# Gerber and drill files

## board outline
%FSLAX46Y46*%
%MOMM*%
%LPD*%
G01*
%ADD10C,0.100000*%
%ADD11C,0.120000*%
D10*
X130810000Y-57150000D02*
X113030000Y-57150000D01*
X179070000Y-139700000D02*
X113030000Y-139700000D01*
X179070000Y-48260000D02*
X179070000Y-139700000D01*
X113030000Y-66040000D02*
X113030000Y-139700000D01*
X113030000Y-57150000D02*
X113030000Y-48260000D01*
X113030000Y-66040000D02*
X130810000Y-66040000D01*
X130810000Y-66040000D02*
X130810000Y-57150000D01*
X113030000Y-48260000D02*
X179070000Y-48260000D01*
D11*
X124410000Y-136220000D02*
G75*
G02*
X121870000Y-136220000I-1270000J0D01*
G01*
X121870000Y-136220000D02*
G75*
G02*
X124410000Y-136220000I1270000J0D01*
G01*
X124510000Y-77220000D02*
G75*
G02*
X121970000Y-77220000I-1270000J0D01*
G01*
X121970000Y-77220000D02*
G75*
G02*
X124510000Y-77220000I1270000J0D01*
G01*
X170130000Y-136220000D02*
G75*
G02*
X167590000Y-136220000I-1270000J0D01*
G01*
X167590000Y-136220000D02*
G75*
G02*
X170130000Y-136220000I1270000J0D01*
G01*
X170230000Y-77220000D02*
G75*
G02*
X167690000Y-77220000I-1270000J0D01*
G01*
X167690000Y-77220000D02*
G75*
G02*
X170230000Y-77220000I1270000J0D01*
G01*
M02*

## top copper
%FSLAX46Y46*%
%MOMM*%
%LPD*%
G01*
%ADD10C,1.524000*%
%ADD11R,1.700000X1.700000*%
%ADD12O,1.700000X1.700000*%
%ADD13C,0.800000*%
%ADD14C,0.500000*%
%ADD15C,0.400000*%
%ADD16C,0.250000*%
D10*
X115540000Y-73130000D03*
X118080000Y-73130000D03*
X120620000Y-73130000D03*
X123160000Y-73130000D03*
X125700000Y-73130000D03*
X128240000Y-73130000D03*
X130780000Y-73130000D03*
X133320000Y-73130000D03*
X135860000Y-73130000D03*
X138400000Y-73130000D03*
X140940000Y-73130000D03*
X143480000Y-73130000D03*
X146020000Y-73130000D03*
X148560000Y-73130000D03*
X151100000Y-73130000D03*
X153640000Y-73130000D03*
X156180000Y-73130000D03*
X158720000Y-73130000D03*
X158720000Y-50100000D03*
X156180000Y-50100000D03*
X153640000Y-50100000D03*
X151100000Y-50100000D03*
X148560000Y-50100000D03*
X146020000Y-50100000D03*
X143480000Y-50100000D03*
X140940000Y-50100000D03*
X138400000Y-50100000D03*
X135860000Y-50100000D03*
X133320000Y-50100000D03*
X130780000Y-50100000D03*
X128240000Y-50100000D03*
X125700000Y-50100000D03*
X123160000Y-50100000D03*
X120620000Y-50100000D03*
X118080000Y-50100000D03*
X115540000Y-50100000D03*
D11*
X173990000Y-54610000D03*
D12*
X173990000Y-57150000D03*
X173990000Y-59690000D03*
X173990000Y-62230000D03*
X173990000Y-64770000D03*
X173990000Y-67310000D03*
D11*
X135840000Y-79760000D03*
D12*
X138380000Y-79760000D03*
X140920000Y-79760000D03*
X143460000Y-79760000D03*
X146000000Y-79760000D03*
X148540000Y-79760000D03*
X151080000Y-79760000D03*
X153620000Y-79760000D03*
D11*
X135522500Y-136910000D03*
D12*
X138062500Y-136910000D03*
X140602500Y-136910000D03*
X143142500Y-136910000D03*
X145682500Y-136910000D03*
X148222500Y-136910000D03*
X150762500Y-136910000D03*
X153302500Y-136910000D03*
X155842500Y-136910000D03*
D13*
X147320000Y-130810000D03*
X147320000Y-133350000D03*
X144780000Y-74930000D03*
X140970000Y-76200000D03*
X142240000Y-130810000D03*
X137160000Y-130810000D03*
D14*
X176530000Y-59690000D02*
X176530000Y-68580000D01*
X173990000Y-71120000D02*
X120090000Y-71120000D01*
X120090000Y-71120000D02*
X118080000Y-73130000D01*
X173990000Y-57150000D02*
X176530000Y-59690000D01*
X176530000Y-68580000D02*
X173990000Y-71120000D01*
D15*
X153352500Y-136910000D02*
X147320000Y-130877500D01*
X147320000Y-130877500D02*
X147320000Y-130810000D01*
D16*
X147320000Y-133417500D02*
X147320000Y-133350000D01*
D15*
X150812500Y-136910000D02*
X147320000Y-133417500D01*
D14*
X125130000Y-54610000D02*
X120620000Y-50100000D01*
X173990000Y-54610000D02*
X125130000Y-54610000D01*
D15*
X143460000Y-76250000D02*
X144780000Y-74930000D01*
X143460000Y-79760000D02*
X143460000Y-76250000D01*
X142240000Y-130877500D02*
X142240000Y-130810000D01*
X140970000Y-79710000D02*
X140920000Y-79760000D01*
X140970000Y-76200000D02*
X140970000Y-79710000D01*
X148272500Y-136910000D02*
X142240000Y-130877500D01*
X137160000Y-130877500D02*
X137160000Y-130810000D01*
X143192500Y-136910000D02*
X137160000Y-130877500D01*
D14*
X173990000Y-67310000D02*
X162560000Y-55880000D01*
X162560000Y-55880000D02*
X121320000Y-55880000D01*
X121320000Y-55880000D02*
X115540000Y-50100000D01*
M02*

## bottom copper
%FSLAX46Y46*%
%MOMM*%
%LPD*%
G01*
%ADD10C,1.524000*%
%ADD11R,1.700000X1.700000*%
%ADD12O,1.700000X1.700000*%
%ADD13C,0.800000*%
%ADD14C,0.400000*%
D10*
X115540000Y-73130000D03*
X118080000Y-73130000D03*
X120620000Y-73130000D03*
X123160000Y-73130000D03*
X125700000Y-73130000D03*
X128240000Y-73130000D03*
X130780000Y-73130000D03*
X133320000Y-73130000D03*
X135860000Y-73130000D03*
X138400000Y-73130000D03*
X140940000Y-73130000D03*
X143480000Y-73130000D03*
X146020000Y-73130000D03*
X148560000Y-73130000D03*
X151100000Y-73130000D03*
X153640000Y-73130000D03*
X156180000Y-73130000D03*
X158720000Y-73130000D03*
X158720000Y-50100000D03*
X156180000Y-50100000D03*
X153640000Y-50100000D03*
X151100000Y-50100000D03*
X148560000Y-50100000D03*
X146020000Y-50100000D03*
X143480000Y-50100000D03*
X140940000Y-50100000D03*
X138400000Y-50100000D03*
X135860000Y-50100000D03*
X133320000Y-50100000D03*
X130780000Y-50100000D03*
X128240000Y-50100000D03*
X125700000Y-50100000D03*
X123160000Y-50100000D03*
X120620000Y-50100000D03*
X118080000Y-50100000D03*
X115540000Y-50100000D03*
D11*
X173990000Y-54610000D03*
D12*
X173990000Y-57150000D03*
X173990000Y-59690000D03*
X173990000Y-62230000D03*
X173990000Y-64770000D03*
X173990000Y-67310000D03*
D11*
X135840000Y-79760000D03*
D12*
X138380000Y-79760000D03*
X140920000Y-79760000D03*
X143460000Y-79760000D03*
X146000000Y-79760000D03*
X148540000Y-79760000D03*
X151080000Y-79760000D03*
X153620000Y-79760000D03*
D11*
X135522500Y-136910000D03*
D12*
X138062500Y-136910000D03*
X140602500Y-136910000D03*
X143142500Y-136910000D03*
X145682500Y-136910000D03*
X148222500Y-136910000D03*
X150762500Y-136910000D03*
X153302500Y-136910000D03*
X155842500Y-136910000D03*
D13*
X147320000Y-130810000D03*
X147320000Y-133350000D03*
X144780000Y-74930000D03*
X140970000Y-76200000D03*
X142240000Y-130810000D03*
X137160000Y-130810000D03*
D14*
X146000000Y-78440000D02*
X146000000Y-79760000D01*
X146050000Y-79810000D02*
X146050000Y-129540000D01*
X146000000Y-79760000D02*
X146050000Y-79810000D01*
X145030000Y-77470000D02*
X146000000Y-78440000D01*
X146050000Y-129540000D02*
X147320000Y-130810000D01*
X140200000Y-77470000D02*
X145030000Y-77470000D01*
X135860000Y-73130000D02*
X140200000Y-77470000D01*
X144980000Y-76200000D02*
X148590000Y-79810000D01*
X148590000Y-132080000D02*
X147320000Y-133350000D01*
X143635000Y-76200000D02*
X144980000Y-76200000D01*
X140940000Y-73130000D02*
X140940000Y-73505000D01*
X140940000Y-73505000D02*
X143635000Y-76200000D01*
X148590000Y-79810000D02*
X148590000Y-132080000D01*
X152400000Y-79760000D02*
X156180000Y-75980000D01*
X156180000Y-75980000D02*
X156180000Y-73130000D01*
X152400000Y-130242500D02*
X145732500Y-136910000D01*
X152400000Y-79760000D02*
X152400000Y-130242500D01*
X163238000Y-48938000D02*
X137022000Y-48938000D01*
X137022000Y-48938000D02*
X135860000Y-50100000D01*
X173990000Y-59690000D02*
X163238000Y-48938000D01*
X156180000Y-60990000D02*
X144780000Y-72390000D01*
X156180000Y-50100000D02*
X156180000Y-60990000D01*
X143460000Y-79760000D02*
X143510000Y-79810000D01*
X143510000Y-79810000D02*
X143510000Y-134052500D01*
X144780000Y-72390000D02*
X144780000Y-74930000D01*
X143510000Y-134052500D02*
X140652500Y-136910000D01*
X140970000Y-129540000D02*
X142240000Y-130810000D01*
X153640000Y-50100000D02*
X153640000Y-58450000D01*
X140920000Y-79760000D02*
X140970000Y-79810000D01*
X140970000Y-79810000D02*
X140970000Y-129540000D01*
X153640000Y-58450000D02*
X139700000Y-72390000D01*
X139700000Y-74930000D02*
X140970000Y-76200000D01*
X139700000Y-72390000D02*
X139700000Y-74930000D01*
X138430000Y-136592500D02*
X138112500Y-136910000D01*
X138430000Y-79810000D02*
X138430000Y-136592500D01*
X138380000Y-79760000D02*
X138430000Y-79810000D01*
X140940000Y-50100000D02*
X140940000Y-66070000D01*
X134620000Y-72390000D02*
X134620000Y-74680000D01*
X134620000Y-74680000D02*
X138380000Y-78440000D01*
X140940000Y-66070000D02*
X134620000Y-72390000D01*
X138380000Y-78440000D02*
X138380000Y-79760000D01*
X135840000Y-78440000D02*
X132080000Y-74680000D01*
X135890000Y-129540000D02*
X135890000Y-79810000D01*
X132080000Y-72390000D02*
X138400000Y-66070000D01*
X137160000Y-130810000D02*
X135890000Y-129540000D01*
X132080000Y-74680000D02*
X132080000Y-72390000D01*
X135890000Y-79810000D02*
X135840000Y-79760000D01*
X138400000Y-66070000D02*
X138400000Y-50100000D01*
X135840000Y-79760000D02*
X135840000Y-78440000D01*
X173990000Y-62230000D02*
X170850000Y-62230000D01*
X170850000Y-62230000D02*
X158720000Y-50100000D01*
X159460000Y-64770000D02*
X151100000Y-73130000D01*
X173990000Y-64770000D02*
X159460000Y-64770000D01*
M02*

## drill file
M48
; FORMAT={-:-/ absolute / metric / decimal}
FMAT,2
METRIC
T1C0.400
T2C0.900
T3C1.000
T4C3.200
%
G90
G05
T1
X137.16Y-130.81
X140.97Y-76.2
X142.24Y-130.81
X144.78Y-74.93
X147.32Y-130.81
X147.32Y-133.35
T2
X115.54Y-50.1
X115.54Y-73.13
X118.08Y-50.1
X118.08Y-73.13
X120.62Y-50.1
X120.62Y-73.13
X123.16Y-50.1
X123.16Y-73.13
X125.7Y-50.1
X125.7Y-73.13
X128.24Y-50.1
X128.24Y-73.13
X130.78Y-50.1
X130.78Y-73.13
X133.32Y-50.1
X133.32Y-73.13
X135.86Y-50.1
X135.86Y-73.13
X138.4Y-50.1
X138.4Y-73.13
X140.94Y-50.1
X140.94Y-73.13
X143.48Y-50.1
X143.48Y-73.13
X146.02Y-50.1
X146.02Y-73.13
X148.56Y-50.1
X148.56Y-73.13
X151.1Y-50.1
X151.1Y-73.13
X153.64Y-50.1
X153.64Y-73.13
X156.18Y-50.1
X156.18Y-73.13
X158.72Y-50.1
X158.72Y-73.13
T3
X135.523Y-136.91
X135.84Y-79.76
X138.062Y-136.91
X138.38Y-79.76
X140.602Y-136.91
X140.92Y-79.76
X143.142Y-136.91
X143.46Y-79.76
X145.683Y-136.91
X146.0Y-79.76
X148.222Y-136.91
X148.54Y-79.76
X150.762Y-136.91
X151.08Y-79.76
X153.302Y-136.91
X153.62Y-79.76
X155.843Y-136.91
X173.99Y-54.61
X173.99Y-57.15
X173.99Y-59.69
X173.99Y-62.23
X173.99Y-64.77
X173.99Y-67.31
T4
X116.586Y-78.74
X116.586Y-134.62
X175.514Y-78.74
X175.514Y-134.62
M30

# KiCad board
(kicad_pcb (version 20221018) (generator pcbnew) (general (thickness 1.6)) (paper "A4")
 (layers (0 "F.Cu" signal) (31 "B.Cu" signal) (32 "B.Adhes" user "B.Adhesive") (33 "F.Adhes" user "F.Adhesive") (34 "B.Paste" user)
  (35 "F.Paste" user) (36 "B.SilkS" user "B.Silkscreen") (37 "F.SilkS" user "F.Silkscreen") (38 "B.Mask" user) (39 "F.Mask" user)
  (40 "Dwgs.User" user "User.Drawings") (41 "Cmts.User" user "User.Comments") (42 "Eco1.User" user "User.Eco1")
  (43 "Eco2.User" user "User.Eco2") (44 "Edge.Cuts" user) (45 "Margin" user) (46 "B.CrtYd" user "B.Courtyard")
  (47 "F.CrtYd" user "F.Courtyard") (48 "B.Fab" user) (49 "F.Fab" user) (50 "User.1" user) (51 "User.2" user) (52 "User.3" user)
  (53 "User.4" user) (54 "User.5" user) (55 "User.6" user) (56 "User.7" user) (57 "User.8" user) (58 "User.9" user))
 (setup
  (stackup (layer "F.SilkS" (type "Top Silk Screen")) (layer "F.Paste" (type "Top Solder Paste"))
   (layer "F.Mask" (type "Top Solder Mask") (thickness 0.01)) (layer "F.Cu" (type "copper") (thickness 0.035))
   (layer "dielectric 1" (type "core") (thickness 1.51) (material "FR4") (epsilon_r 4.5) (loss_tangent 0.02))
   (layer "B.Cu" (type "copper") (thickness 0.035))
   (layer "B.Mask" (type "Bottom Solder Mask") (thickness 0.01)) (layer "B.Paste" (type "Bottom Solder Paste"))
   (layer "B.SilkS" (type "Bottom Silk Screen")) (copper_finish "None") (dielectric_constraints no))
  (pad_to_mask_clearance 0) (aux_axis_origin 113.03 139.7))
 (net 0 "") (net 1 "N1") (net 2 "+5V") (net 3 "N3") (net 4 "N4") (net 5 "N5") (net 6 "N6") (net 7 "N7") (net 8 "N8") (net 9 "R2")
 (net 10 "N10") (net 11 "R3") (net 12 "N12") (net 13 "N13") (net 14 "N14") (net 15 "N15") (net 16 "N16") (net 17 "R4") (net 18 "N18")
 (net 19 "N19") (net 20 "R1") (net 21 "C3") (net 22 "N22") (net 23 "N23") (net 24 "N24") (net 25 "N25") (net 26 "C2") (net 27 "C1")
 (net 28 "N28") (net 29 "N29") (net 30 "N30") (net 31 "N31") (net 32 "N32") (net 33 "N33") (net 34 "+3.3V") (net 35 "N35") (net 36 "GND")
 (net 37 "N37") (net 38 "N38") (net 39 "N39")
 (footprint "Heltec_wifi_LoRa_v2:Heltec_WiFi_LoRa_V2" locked (layer "F.Cu") (at 140.94 61.615 90)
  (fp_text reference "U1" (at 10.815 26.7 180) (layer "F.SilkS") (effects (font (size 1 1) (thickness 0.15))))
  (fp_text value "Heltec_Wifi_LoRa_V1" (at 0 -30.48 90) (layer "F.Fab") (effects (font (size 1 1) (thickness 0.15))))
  (pad "1" thru_hole circle locked (at -11.515 -25.4 90) (size 1.524 1.524) (drill 0.9) (layers "*.Cu" "*.Mask") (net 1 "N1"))
  (pad "2" thru_hole circle locked (at -11.515 -22.86 90) (size 1.524 1.524) (drill 0.9) (layers "*.Cu" "*.Mask") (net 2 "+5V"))
  (pad "3" thru_hole circle locked (at -11.515 -20.32 90) (size 1.524 1.524) (drill 0.9) (layers "*.Cu" "*.Mask") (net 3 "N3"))
  (pad "4" thru_hole circle locked (at -11.515 -17.78 90) (size 1.524 1.524) (drill 0.9) (layers "*.Cu" "*.Mask") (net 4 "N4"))
  (pad "5" thru_hole circle locked (at -11.515 -15.24 90) (size 1.524 1.524) (drill 0.9) (layers "*.Cu" "*.Mask") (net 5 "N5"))
  (pad "6" thru_hole circle locked (at -11.515 -12.7 90) (size 1.524 1.524) (drill 0.9) (layers "*.Cu" "*.Mask") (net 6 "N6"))
  (pad "7" thru_hole circle locked (at -11.515 -10.16 90) (size 1.524 1.524) (drill 0.9) (layers "*.Cu" "*.Mask") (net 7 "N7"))
  (pad "8" thru_hole circle locked (at -11.515 -7.62 90) (size 1.524 1.524) (drill 0.9) (layers "*.Cu" "*.Mask") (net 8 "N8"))
  (pad "9" thru_hole circle locked (at -11.515 -5.08 90) (size 1.524 1.524) (drill 0.9) (layers "*.Cu" "*.Mask") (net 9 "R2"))
  (pad "10" thru_hole circle locked (at -11.515 -2.54 90) (size 1.524 1.524) (drill 0.9) (layers "*.Cu" "*.Mask") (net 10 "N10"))
  (pad "11" thru_hole circle locked (at -11.515 0 90) (size 1.524 1.524) (drill 0.9) (layers "*.Cu" "*.Mask") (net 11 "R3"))
  (pad "12" thru_hole circle locked (at -11.515 2.54 90) (size 1.524 1.524) (drill 0.9) (layers "*.Cu" "*.Mask") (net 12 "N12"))
  (pad "13" thru_hole circle locked (at -11.515 5.08 90) (size 1.524 1.524) (drill 0.9) (layers "*.Cu" "*.Mask") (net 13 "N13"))
  (pad "14" thru_hole circle locked (at -11.515 7.62 90) (size 1.524 1.524) (drill 0.9) (layers "*.Cu" "*.Mask") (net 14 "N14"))
  (pad "15" thru_hole circle locked (at -11.515 10.16 90) (size 1.524 1.524) (drill 0.9) (layers "*.Cu" "*.Mask") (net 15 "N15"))
  (pad "16" thru_hole circle locked (at -11.515 12.7 90) (size 1.524 1.524) (drill 0.9) (layers "*.Cu" "*.Mask") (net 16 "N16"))
  (pad "17" thru_hole circle locked (at -11.515 15.24 90) (size 1.524 1.524) (drill 0.9) (layers "*.Cu" "*.Mask") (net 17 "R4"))
  (pad "18" thru_hole circle locked (at -11.515 17.78 90) (size 1.524 1.524) (drill 0.9) (layers "*.Cu" "*.Mask") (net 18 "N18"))
  (pad "19" thru_hole circle locked (at 11.515 17.78 90) (size 1.524 1.524) (drill 0.9) (layers "*.Cu" "*.Mask") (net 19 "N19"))
  (pad "20" thru_hole circle locked (at 11.515 15.24 90) (size 1.524 1.524) (drill 0.9) (layers "*.Cu" "*.Mask") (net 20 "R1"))
  (pad "21" thru_hole circle locked (at 11.515 12.7 90) (size 1.524 1.524) (drill 0.9) (layers "*.Cu" "*.Mask") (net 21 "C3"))
  (pad "22" thru_hole circle locked (at 11.515 10.16 90) (size 1.524 1.524) (drill 0.9) (layers "*.Cu" "*.Mask") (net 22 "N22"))
  (pad "23" thru_hole circle locked (at 11.515 7.62 90) (size 1.524 1.524) (drill 0.9) (layers "*.Cu" "*.Mask") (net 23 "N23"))
  (pad "24" thru_hole circle locked (at 11.515 5.08 90) (size 1.524 1.524) (drill 0.9) (layers "*.Cu" "*.Mask") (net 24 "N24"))
  (pad "25" thru_hole circle locked (at 11.515 2.54 90) (size 1.524 1.524) (drill 0.9) (layers "*.Cu" "*.Mask") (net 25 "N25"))
  (pad "26" thru_hole circle locked (at 11.515 0 90) (size 1.524 1.524) (drill 0.9) (layers "*.Cu" "*.Mask") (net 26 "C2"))
  (pad "27" thru_hole circle locked (at 11.515 -2.54 90) (size 1.524 1.524) (drill 0.9) (layers "*.Cu" "*.Mask") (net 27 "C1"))
  (pad "28" thru_hole circle locked (at 11.515 -5.08 90) (size 1.524 1.524) (drill 0.9) (layers "*.Cu" "*.Mask") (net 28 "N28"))
  (pad "29" thru_hole circle locked (at 11.515 -7.62 90) (size 1.524 1.524) (drill 0.9) (layers "*.Cu" "*.Mask") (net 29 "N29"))
  (pad "30" thru_hole circle locked (at 11.515 -10.16 90) (size 1.524 1.524) (drill 0.9) (layers "*.Cu" "*.Mask") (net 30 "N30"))
  (pad "31" thru_hole circle locked (at 11.515 -12.7 90) (size 1.524 1.524) (drill 0.9) (layers "*.Cu" "*.Mask") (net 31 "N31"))
  (pad "32" thru_hole circle locked (at 11.515 -15.24 90) (size 1.524 1.524) (drill 0.9) (layers "*.Cu" "*.Mask") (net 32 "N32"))
  (pad "33" thru_hole circle locked (at 11.515 -17.78 90) (size 1.524 1.524) (drill 0.9) (layers "*.Cu" "*.Mask") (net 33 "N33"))
  (pad "34" thru_hole circle locked (at 11.515 -20.32 90) (size 1.524 1.524) (drill 0.9) (layers "*.Cu" "*.Mask") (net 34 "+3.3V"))
  (pad "35" thru_hole circle locked (at 11.515 -22.86 90) (size 1.524 1.524) (drill 0.9) (layers "*.Cu" "*.Mask") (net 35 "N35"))
  (pad "36" thru_hole circle locked (at 11.515 -25.4 90) (size 1.524 1.524) (drill 0.9) (layers "*.Cu" "*.Mask") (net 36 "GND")))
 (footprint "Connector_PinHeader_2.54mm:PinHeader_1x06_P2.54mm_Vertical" (layer "F.Cu") (at 173.99 54.61)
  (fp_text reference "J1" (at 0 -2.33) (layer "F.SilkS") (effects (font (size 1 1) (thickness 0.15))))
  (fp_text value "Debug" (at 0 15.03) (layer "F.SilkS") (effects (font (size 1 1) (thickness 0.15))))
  (pad "1" thru_hole rect (at 0 0) (size 1.7 1.7) (drill 1) (layers "*.Cu" "*.Mask") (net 34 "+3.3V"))
  (pad "2" thru_hole oval (at 0 2.54) (size 1.7 1.7) (drill 1) (layers "*.Cu" "*.Mask") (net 2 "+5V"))
  (pad "3" thru_hole oval (at 0 5.08) (size 1.7 1.7) (drill 1) (layers "*.Cu" "*.Mask") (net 28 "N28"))
  (pad "4" thru_hole oval (at 0 7.62) (size 1.7 1.7) (drill 1) (layers "*.Cu" "*.Mask") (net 19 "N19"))
  (pad "5" thru_hole oval (at 0 10.16) (size 1.7 1.7) (drill 1) (layers "*.Cu" "*.Mask") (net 15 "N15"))
  (pad "6" thru_hole oval (at 0 12.7) (size 1.7 1.7) (drill 1) (layers "*.Cu" "*.Mask") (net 36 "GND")))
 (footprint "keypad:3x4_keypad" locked (layer "F.Cu") (at 135.84 79.76)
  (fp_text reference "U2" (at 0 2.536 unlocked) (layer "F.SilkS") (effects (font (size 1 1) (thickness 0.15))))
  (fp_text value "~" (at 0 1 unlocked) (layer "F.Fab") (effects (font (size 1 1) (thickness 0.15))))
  (fp_circle (center -12.7 56.46) (end -11.43 56.46) (stroke (width 0.12) (type default)) (fill none) (layer "Edge.Cuts"))
  (fp_circle (center -12.6 -2.54) (end -12.6 -3.81) (stroke (width 0.12) (type default)) (fill none) (layer "Edge.Cuts"))
  (fp_circle (center 33.02 56.46) (end 34.29 56.46) (stroke (width 0.12) (type default)) (fill none) (layer "Edge.Cuts"))
  (fp_circle (center 33.12 -2.54) (end 31.85 -2.54) (stroke (width 0.12) (type default)) (fill none) (layer "Edge.Cuts"))
  (pad "A1" thru_hole rect locked (at 0 0 90) (size 1.7 1.7) (drill 1) (layers "*.Cu" "*.Mask") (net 27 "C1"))
  (pad "A2" thru_hole oval locked (at 2.54 0 90) (size 1.7 1.7) (drill 1) (layers "*.Cu" "*.Mask") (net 26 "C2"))
  (pad "A3" thru_hole oval locked (at 5.08 0 90) (size 1.7 1.7) (drill 1) (layers "*.Cu" "*.Mask") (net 21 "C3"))
  (pad "A4" thru_hole oval locked (at 7.62 0 90) (size 1.7 1.7) (drill 1) (layers "*.Cu" "*.Mask") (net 20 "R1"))
  (pad "A5" thru_hole oval locked (at 10.16 0 90) (size 1.7 1.7) (drill 1) (layers "*.Cu" "*.Mask") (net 9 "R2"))
  (pad "A6" thru_hole oval locked (at 12.7 0 90) (size 1.7 1.7) (drill 1) (layers "*.Cu" "*.Mask") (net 11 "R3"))
  (pad "A7" thru_hole oval locked (at 15.24 0 90) (size 1.7 1.7) (drill 1) (layers "*.Cu" "*.Mask") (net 17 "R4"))
  (pad "A8" thru_hole oval locked (at 17.78 0 90) (size 1.7 1.7) (drill 1) (layers "*.Cu" "*.Mask") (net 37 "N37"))
  (pad "B1" thru_hole rect locked (at -0.3175 57.15 90) (size 1.7 1.7) (drill 1) (layers "*.Cu" "*.Mask") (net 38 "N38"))
  (pad "B2" thru_hole oval locked (at 2.2225 57.15 90) (size 1.7 1.7) (drill 1) (layers "*.Cu" "*.Mask") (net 26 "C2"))
  (pad "B3" thru_hole oval locked (at 4.7625 57.15 90) (size 1.7 1.7) (drill 1) (layers "*.Cu" "*.Mask") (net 20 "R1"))
  (pad "B4" thru_hole oval locked (at 7.3025 57.15 90) (size 1.7 1.7) (drill 1) (layers "*.Cu" "*.Mask") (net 27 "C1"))
  (pad "B5" thru_hole oval locked (at 9.8425 57.15 90) (size 1.7 1.7) (drill 1) (layers "*.Cu" "*.Mask") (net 17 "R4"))
  (pad "B6" thru_hole oval locked (at 12.3825 57.15 90) (size 1.7 1.7) (drill 1) (layers "*.Cu" "*.Mask") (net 21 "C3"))
  (pad "B7" thru_hole oval locked (at 14.9225 57.15 90) (size 1.7 1.7) (drill 1) (layers "*.Cu" "*.Mask") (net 11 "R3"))
  (pad "B8" thru_hole oval locked (at 17.4625 57.15 90) (size 1.7 1.7) (drill 1) (layers "*.Cu" "*.Mask") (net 9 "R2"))
  (pad "B9" thru_hole oval locked (at 20.0025 57.15 90) (size 1.7 1.7) (drill 1) (layers "*.Cu" "*.Mask") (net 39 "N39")))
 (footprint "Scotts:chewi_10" (layer "F.Cu") (at 116.586 102.362 90)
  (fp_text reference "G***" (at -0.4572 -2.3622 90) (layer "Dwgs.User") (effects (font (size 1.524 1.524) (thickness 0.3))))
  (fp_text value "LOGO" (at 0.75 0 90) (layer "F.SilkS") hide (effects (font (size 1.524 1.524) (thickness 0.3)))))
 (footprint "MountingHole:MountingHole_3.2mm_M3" (layer "F.Cu") (at 116.586 134.62)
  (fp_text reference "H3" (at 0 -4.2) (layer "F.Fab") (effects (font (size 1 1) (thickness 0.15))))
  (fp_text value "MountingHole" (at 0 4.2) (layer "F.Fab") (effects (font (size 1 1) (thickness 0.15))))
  (pad "" np_thru_hole circle (at 0 0) (size 3.2 3.2) (drill 3.2) (layers "*.Cu" "*.Mask")))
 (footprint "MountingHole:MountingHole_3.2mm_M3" (layer "F.Cu") (at 116.586 78.74)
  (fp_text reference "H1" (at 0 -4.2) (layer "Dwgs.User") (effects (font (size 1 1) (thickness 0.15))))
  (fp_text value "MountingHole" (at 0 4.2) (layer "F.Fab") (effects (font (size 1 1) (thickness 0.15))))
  (pad "" np_thru_hole circle (at 0 0) (size 3.2 3.2) (drill 3.2) (layers "*.Cu" "*.Mask")))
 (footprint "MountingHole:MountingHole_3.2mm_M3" (layer "F.Cu") (at 175.514 78.74)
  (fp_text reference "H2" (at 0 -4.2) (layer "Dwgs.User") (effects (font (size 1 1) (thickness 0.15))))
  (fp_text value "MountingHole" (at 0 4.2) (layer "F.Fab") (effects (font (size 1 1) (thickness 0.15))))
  (pad "" np_thru_hole circle (at 0 0) (size 3.2 3.2) (drill 3.2) (layers "*.Cu" "*.Mask")))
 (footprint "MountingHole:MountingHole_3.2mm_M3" (layer "F.Cu") (at 175.514 134.62)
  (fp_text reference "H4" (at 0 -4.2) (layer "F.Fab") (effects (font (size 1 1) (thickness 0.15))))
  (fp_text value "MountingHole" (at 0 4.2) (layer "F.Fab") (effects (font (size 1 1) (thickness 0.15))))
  (pad "" np_thru_hole circle (at 0 0) (size 3.2 3.2) (drill 3.2) (layers "*.Cu" "*.Mask")))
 (gr_line (start 130.81 57.15) (end 113.03 57.15) (stroke (width 0.1) (type default)) (layer "Edge.Cuts"))
 (gr_line (start 179.07 139.7) (end 113.03 139.7) (stroke (width 0.1) (type default)) (layer "Edge.Cuts"))
 (gr_line (start 179.07 48.26) (end 179.07 139.7) (stroke (width 0.1) (type default)) (layer "Edge.Cuts"))
 (gr_line (start 113.03 66.04) (end 113.03 139.7) (stroke (width 0.1) (type default)) (layer "Edge.Cuts"))
 (gr_line (start 113.03 57.15) (end 113.03 48.26) (stroke (width 0.1) (type default)) (layer "Edge.Cuts"))
 (gr_line (start 113.03 66.04) (end 130.81 66.04) (stroke (width 0.1) (type default)) (layer "Edge.Cuts"))
 (gr_line (start 130.81 66.04) (end 130.81 57.15) (stroke (width 0.1) (type default)) (layer "Edge.Cuts"))
 (gr_line (start 113.03 48.26) (end 179.07 48.26) (stroke (width 0.1) (type default)) (layer "Edge.Cuts"))
 (segment (start 176.53 59.69) (end 176.53 68.58) (width 0.5) (layer "F.Cu") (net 2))
 (segment (start 173.99 71.12) (end 120.09 71.12) (width 0.5) (layer "F.Cu") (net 2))
 (segment (start 120.09 71.12) (end 118.08 73.13) (width 0.5) (layer "F.Cu") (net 2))
 (segment (start 173.99 57.15) (end 176.53 59.69) (width 0.5) (layer "F.Cu") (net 2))
 (segment (start 176.53 68.58) (end 173.99 71.12) (width 0.5) (layer "F.Cu") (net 2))
 (segment (start 153.3525 136.91) (end 147.32 130.8775) (width 0.4) (layer "F.Cu") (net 9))
 (segment (start 147.32 130.8775) (end 147.32 130.81) (width 0.4) (layer "F.Cu") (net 9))
 (via (at 147.32 130.81) (size 0.8) (drill 0.4) (layers "F.Cu" "B.Cu") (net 9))
 (segment (start 146 78.44) (end 146 79.76) (width 0.4) (layer "B.Cu") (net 9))
 (segment (start 146.05 79.81) (end 146.05 129.54) (width 0.4) (layer "B.Cu") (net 9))
 (segment (start 146 79.76) (end 146.05 79.81) (width 0.4) (layer "B.Cu") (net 9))
 (segment (start 145.03 77.47) (end 146 78.44) (width 0.4) (layer "B.Cu") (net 9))
 (segment (start 146.05 129.54) (end 147.32 130.81) (width 0.4) (layer "B.Cu") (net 9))
 (segment (start 140.2 77.47) (end 145.03 77.47) (width 0.4) (layer "B.Cu") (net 9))
 (segment (start 135.86 73.13) (end 140.2 77.47) (width 0.4) (layer "B.Cu") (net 9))
 (segment (start 147.32 133.4175) (end 147.32 133.35) (width 0.25) (layer "F.Cu") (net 11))
 (segment (start 150.8125 136.91) (end 147.32 133.4175) (width 0.4) (layer "F.Cu") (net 11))
 (via (at 147.32 133.35) (size 0.8) (drill 0.4) (layers "F.Cu" "B.Cu") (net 11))
 (segment (start 144.98 76.2) (end 148.59 79.81) (width 0.4) (layer "B.Cu") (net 11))
 (segment (start 148.59 132.08) (end 147.32 133.35) (width 0.4) (layer "B.Cu") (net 11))
 (segment (start 143.635 76.2) (end 144.98 76.2) (width 0.4) (layer "B.Cu") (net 11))
 (segment (start 140.94 73.13) (end 140.94 73.505) (width 0.4) (layer "B.Cu") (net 11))
 (segment (start 140.94 73.505) (end 143.635 76.2) (width 0.4) (layer "B.Cu") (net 11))
 (segment (start 148.59 79.81) (end 148.59 132.08) (width 0.4) (layer "B.Cu") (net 11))
 (segment (start 125.13 54.61) (end 120.62 50.1) (width 0.5) (layer "F.Cu") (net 34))
 (segment (start 173.99 54.61) (end 125.13 54.61) (width 0.5) (layer "F.Cu") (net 34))
 (segment (start 152.4 79.76) (end 156.18 75.98) (width 0.4) (layer "B.Cu") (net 17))
 (segment (start 156.18 75.98) (end 156.18 73.13) (width 0.4) (layer "B.Cu") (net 17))
 (segment (start 152.4 130.2425) (end 145.7325 136.91) (width 0.4) (layer "B.Cu") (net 17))
 (segment (start 152.4 79.76) (end 152.4 130.2425) (width 0.4) (layer "B.Cu") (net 17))
 (segment (start 163.238 48.938) (end 137.022 48.938) (width 0.4) (layer "B.Cu") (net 28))
 (segment (start 137.022 48.938) (end 135.86 50.1) (width 0.4) (layer "B.Cu") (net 28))
 (segment (start 173.99 59.69) (end 163.238 48.938) (width 0.4) (layer "B.Cu") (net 28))
 (segment (start 143.46 76.25) (end 144.78 74.93) (width 0.4) (layer "F.Cu") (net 20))
 (segment (start 143.46 79.76) (end 143.46 76.25) (width 0.4) (layer "F.Cu") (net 20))
 (via (at 144.78 74.93) (size 0.8) (drill 0.4) (layers "F.Cu" "B.Cu") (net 20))
 (segment (start 156.18 60.99) (end 144.78 72.39) (width 0.4) (layer "B.Cu") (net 20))
 (segment (start 156.18 50.1) (end 156.18 60.99) (width 0.4) (layer "B.Cu") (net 20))
 (segment (start 143.46 79.76) (end 143.51 79.81) (width 0.4) (layer "B.Cu") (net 20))
 (segment (start 143.51 79.81) (end 143.51 134.0525) (width 0.4) (layer "B.Cu") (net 20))
 (segment (start 144.78 72.39) (end 144.78 74.93) (width 0.4) (layer "B.Cu") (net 20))
 (segment (start 143.51 134.0525) (end 140.6525 136.91) (width 0.4) (layer "B.Cu") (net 20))
 (segment (start 142.24 130.8775) (end 142.24 130.81) (width 0.4) (layer "F.Cu") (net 21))
 (segment (start 140.97 79.71) (end 140.92 79.76) (width 0.4) (layer "F.Cu") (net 21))
 (segment (start 140.97 76.2) (end 140.97 79.71) (width 0.4) (layer "F.Cu") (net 21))
 (segment (start 148.2725 136.91) (end 142.24 130.8775) (width 0.4) (layer "F.Cu") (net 21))
 (via (at 140.97 76.2) (size 0.8) (drill 0.4) (layers "F.Cu" "B.Cu") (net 21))
 (via (at 142.24 130.81) (size 0.8) (drill 0.4) (layers "F.Cu" "B.Cu") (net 21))
 (segment (start 140.97 129.54) (end 142.24 130.81) (width 0.4) (layer "B.Cu") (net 21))
 (segment (start 153.64 50.1) (end 153.64 58.45) (width 0.4) (layer "B.Cu") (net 21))
 (segment (start 140.92 79.76) (end 140.97 79.81) (width 0.4) (layer "B.Cu") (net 21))
 (segment (start 140.97 79.81) (end 140.97 129.54) (width 0.4) (layer "B.Cu") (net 21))
 (segment (start 153.64 58.45) (end 139.7 72.39) (width 0.4) (layer "B.Cu") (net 21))
 (segment (start 139.7 74.93) (end 140.97 76.2) (width 0.4) (layer "B.Cu") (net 21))
 (segment (start 139.7 72.39) (end 139.7 74.93) (width 0.4) (layer "B.Cu") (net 21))
 (segment (start 138.43 136.5925) (end 138.1125 136.91) (width 0.4) (layer "B.Cu") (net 26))
 (segment (start 138.43 79.81) (end 138.43 136.5925) (width 0.4) (layer "B.Cu") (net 26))
 (segment (start 138.38 79.76) (end 138.43 79.81) (width 0.4) (layer "B.Cu") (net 26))
 (segment (start 140.94 50.1) (end 140.94 66.07) (width 0.4) (layer "B.Cu") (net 26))
 (segment (start 134.62 72.39) (end 134.62 74.68) (width 0.4) (layer "B.Cu") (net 26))
 (segment (start 134.62 74.68) (end 138.38 78.44) (width 0.4) (layer "B.Cu") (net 26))
 (segment (start 140.94 66.07) (end 134.62 72.39) (width 0.4) (layer "B.Cu") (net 26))
 (segment (start 138.38 78.44) (end 138.38 79.76) (width 0.4) (layer "B.Cu") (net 26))
 (segment (start 137.16 130.8775) (end 137.16 130.81) (width 0.4) (layer "F.Cu") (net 27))
 (segment (start 143.1925 136.91) (end 137.16 130.8775) (width 0.4) (layer "F.Cu") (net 27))
 (via (at 137.16 130.81) (size 0.8) (drill 0.4) (layers "F.Cu" "B.Cu") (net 27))
 (segment (start 135.84 78.44) (end 132.08 74.68) (width 0.4) (layer "B.Cu") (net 27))
 (segment (start 135.89 129.54) (end 135.89 79.81) (width 0.4) (layer "B.Cu") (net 27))
 (segment (start 132.08 72.39) (end 138.4 66.07) (width 0.4) (layer "B.Cu") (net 27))
 (segment (start 137.16 130.81) (end 135.89 129.54) (width 0.4) (layer "B.Cu") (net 27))
 (segment (start 132.08 74.68) (end 132.08 72.39) (width 0.4) (layer "B.Cu") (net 27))
 (segment (start 135.89 79.81) (end 135.84 79.76) (width 0.4) (layer "B.Cu") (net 27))
 (segment (start 138.4 66.07) (end 138.4 50.1) (width 0.4) (layer "B.Cu") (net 27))
 (segment (start 135.84 79.76) (end 135.84 78.44) (width 0.4) (layer "B.Cu") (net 27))
 (segment (start 173.99 62.23) (end 170.85 62.23) (width 0.4) (layer "B.Cu") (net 19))
 (segment (start 170.85 62.23) (end 158.72 50.1) (width 0.4) (layer "B.Cu") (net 19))
 (segment (start 159.46 64.77) (end 151.1 73.13) (width 0.4) (layer "B.Cu") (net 15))
 (segment (start 173.99 64.77) (end 159.46 64.77) (width 0.4) (layer "B.Cu") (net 15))
 (segment (start 173.99 67.31) (end 162.56 55.88) (width 0.5) (layer "F.Cu") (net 36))
 (segment (start 162.56 55.88) (end 121.32 55.88) (width 0.5) (layer "F.Cu") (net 36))
 (segment (start 121.32 55.88) (end 115.54 50.1) (width 0.5) (layer "F.Cu") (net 36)))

